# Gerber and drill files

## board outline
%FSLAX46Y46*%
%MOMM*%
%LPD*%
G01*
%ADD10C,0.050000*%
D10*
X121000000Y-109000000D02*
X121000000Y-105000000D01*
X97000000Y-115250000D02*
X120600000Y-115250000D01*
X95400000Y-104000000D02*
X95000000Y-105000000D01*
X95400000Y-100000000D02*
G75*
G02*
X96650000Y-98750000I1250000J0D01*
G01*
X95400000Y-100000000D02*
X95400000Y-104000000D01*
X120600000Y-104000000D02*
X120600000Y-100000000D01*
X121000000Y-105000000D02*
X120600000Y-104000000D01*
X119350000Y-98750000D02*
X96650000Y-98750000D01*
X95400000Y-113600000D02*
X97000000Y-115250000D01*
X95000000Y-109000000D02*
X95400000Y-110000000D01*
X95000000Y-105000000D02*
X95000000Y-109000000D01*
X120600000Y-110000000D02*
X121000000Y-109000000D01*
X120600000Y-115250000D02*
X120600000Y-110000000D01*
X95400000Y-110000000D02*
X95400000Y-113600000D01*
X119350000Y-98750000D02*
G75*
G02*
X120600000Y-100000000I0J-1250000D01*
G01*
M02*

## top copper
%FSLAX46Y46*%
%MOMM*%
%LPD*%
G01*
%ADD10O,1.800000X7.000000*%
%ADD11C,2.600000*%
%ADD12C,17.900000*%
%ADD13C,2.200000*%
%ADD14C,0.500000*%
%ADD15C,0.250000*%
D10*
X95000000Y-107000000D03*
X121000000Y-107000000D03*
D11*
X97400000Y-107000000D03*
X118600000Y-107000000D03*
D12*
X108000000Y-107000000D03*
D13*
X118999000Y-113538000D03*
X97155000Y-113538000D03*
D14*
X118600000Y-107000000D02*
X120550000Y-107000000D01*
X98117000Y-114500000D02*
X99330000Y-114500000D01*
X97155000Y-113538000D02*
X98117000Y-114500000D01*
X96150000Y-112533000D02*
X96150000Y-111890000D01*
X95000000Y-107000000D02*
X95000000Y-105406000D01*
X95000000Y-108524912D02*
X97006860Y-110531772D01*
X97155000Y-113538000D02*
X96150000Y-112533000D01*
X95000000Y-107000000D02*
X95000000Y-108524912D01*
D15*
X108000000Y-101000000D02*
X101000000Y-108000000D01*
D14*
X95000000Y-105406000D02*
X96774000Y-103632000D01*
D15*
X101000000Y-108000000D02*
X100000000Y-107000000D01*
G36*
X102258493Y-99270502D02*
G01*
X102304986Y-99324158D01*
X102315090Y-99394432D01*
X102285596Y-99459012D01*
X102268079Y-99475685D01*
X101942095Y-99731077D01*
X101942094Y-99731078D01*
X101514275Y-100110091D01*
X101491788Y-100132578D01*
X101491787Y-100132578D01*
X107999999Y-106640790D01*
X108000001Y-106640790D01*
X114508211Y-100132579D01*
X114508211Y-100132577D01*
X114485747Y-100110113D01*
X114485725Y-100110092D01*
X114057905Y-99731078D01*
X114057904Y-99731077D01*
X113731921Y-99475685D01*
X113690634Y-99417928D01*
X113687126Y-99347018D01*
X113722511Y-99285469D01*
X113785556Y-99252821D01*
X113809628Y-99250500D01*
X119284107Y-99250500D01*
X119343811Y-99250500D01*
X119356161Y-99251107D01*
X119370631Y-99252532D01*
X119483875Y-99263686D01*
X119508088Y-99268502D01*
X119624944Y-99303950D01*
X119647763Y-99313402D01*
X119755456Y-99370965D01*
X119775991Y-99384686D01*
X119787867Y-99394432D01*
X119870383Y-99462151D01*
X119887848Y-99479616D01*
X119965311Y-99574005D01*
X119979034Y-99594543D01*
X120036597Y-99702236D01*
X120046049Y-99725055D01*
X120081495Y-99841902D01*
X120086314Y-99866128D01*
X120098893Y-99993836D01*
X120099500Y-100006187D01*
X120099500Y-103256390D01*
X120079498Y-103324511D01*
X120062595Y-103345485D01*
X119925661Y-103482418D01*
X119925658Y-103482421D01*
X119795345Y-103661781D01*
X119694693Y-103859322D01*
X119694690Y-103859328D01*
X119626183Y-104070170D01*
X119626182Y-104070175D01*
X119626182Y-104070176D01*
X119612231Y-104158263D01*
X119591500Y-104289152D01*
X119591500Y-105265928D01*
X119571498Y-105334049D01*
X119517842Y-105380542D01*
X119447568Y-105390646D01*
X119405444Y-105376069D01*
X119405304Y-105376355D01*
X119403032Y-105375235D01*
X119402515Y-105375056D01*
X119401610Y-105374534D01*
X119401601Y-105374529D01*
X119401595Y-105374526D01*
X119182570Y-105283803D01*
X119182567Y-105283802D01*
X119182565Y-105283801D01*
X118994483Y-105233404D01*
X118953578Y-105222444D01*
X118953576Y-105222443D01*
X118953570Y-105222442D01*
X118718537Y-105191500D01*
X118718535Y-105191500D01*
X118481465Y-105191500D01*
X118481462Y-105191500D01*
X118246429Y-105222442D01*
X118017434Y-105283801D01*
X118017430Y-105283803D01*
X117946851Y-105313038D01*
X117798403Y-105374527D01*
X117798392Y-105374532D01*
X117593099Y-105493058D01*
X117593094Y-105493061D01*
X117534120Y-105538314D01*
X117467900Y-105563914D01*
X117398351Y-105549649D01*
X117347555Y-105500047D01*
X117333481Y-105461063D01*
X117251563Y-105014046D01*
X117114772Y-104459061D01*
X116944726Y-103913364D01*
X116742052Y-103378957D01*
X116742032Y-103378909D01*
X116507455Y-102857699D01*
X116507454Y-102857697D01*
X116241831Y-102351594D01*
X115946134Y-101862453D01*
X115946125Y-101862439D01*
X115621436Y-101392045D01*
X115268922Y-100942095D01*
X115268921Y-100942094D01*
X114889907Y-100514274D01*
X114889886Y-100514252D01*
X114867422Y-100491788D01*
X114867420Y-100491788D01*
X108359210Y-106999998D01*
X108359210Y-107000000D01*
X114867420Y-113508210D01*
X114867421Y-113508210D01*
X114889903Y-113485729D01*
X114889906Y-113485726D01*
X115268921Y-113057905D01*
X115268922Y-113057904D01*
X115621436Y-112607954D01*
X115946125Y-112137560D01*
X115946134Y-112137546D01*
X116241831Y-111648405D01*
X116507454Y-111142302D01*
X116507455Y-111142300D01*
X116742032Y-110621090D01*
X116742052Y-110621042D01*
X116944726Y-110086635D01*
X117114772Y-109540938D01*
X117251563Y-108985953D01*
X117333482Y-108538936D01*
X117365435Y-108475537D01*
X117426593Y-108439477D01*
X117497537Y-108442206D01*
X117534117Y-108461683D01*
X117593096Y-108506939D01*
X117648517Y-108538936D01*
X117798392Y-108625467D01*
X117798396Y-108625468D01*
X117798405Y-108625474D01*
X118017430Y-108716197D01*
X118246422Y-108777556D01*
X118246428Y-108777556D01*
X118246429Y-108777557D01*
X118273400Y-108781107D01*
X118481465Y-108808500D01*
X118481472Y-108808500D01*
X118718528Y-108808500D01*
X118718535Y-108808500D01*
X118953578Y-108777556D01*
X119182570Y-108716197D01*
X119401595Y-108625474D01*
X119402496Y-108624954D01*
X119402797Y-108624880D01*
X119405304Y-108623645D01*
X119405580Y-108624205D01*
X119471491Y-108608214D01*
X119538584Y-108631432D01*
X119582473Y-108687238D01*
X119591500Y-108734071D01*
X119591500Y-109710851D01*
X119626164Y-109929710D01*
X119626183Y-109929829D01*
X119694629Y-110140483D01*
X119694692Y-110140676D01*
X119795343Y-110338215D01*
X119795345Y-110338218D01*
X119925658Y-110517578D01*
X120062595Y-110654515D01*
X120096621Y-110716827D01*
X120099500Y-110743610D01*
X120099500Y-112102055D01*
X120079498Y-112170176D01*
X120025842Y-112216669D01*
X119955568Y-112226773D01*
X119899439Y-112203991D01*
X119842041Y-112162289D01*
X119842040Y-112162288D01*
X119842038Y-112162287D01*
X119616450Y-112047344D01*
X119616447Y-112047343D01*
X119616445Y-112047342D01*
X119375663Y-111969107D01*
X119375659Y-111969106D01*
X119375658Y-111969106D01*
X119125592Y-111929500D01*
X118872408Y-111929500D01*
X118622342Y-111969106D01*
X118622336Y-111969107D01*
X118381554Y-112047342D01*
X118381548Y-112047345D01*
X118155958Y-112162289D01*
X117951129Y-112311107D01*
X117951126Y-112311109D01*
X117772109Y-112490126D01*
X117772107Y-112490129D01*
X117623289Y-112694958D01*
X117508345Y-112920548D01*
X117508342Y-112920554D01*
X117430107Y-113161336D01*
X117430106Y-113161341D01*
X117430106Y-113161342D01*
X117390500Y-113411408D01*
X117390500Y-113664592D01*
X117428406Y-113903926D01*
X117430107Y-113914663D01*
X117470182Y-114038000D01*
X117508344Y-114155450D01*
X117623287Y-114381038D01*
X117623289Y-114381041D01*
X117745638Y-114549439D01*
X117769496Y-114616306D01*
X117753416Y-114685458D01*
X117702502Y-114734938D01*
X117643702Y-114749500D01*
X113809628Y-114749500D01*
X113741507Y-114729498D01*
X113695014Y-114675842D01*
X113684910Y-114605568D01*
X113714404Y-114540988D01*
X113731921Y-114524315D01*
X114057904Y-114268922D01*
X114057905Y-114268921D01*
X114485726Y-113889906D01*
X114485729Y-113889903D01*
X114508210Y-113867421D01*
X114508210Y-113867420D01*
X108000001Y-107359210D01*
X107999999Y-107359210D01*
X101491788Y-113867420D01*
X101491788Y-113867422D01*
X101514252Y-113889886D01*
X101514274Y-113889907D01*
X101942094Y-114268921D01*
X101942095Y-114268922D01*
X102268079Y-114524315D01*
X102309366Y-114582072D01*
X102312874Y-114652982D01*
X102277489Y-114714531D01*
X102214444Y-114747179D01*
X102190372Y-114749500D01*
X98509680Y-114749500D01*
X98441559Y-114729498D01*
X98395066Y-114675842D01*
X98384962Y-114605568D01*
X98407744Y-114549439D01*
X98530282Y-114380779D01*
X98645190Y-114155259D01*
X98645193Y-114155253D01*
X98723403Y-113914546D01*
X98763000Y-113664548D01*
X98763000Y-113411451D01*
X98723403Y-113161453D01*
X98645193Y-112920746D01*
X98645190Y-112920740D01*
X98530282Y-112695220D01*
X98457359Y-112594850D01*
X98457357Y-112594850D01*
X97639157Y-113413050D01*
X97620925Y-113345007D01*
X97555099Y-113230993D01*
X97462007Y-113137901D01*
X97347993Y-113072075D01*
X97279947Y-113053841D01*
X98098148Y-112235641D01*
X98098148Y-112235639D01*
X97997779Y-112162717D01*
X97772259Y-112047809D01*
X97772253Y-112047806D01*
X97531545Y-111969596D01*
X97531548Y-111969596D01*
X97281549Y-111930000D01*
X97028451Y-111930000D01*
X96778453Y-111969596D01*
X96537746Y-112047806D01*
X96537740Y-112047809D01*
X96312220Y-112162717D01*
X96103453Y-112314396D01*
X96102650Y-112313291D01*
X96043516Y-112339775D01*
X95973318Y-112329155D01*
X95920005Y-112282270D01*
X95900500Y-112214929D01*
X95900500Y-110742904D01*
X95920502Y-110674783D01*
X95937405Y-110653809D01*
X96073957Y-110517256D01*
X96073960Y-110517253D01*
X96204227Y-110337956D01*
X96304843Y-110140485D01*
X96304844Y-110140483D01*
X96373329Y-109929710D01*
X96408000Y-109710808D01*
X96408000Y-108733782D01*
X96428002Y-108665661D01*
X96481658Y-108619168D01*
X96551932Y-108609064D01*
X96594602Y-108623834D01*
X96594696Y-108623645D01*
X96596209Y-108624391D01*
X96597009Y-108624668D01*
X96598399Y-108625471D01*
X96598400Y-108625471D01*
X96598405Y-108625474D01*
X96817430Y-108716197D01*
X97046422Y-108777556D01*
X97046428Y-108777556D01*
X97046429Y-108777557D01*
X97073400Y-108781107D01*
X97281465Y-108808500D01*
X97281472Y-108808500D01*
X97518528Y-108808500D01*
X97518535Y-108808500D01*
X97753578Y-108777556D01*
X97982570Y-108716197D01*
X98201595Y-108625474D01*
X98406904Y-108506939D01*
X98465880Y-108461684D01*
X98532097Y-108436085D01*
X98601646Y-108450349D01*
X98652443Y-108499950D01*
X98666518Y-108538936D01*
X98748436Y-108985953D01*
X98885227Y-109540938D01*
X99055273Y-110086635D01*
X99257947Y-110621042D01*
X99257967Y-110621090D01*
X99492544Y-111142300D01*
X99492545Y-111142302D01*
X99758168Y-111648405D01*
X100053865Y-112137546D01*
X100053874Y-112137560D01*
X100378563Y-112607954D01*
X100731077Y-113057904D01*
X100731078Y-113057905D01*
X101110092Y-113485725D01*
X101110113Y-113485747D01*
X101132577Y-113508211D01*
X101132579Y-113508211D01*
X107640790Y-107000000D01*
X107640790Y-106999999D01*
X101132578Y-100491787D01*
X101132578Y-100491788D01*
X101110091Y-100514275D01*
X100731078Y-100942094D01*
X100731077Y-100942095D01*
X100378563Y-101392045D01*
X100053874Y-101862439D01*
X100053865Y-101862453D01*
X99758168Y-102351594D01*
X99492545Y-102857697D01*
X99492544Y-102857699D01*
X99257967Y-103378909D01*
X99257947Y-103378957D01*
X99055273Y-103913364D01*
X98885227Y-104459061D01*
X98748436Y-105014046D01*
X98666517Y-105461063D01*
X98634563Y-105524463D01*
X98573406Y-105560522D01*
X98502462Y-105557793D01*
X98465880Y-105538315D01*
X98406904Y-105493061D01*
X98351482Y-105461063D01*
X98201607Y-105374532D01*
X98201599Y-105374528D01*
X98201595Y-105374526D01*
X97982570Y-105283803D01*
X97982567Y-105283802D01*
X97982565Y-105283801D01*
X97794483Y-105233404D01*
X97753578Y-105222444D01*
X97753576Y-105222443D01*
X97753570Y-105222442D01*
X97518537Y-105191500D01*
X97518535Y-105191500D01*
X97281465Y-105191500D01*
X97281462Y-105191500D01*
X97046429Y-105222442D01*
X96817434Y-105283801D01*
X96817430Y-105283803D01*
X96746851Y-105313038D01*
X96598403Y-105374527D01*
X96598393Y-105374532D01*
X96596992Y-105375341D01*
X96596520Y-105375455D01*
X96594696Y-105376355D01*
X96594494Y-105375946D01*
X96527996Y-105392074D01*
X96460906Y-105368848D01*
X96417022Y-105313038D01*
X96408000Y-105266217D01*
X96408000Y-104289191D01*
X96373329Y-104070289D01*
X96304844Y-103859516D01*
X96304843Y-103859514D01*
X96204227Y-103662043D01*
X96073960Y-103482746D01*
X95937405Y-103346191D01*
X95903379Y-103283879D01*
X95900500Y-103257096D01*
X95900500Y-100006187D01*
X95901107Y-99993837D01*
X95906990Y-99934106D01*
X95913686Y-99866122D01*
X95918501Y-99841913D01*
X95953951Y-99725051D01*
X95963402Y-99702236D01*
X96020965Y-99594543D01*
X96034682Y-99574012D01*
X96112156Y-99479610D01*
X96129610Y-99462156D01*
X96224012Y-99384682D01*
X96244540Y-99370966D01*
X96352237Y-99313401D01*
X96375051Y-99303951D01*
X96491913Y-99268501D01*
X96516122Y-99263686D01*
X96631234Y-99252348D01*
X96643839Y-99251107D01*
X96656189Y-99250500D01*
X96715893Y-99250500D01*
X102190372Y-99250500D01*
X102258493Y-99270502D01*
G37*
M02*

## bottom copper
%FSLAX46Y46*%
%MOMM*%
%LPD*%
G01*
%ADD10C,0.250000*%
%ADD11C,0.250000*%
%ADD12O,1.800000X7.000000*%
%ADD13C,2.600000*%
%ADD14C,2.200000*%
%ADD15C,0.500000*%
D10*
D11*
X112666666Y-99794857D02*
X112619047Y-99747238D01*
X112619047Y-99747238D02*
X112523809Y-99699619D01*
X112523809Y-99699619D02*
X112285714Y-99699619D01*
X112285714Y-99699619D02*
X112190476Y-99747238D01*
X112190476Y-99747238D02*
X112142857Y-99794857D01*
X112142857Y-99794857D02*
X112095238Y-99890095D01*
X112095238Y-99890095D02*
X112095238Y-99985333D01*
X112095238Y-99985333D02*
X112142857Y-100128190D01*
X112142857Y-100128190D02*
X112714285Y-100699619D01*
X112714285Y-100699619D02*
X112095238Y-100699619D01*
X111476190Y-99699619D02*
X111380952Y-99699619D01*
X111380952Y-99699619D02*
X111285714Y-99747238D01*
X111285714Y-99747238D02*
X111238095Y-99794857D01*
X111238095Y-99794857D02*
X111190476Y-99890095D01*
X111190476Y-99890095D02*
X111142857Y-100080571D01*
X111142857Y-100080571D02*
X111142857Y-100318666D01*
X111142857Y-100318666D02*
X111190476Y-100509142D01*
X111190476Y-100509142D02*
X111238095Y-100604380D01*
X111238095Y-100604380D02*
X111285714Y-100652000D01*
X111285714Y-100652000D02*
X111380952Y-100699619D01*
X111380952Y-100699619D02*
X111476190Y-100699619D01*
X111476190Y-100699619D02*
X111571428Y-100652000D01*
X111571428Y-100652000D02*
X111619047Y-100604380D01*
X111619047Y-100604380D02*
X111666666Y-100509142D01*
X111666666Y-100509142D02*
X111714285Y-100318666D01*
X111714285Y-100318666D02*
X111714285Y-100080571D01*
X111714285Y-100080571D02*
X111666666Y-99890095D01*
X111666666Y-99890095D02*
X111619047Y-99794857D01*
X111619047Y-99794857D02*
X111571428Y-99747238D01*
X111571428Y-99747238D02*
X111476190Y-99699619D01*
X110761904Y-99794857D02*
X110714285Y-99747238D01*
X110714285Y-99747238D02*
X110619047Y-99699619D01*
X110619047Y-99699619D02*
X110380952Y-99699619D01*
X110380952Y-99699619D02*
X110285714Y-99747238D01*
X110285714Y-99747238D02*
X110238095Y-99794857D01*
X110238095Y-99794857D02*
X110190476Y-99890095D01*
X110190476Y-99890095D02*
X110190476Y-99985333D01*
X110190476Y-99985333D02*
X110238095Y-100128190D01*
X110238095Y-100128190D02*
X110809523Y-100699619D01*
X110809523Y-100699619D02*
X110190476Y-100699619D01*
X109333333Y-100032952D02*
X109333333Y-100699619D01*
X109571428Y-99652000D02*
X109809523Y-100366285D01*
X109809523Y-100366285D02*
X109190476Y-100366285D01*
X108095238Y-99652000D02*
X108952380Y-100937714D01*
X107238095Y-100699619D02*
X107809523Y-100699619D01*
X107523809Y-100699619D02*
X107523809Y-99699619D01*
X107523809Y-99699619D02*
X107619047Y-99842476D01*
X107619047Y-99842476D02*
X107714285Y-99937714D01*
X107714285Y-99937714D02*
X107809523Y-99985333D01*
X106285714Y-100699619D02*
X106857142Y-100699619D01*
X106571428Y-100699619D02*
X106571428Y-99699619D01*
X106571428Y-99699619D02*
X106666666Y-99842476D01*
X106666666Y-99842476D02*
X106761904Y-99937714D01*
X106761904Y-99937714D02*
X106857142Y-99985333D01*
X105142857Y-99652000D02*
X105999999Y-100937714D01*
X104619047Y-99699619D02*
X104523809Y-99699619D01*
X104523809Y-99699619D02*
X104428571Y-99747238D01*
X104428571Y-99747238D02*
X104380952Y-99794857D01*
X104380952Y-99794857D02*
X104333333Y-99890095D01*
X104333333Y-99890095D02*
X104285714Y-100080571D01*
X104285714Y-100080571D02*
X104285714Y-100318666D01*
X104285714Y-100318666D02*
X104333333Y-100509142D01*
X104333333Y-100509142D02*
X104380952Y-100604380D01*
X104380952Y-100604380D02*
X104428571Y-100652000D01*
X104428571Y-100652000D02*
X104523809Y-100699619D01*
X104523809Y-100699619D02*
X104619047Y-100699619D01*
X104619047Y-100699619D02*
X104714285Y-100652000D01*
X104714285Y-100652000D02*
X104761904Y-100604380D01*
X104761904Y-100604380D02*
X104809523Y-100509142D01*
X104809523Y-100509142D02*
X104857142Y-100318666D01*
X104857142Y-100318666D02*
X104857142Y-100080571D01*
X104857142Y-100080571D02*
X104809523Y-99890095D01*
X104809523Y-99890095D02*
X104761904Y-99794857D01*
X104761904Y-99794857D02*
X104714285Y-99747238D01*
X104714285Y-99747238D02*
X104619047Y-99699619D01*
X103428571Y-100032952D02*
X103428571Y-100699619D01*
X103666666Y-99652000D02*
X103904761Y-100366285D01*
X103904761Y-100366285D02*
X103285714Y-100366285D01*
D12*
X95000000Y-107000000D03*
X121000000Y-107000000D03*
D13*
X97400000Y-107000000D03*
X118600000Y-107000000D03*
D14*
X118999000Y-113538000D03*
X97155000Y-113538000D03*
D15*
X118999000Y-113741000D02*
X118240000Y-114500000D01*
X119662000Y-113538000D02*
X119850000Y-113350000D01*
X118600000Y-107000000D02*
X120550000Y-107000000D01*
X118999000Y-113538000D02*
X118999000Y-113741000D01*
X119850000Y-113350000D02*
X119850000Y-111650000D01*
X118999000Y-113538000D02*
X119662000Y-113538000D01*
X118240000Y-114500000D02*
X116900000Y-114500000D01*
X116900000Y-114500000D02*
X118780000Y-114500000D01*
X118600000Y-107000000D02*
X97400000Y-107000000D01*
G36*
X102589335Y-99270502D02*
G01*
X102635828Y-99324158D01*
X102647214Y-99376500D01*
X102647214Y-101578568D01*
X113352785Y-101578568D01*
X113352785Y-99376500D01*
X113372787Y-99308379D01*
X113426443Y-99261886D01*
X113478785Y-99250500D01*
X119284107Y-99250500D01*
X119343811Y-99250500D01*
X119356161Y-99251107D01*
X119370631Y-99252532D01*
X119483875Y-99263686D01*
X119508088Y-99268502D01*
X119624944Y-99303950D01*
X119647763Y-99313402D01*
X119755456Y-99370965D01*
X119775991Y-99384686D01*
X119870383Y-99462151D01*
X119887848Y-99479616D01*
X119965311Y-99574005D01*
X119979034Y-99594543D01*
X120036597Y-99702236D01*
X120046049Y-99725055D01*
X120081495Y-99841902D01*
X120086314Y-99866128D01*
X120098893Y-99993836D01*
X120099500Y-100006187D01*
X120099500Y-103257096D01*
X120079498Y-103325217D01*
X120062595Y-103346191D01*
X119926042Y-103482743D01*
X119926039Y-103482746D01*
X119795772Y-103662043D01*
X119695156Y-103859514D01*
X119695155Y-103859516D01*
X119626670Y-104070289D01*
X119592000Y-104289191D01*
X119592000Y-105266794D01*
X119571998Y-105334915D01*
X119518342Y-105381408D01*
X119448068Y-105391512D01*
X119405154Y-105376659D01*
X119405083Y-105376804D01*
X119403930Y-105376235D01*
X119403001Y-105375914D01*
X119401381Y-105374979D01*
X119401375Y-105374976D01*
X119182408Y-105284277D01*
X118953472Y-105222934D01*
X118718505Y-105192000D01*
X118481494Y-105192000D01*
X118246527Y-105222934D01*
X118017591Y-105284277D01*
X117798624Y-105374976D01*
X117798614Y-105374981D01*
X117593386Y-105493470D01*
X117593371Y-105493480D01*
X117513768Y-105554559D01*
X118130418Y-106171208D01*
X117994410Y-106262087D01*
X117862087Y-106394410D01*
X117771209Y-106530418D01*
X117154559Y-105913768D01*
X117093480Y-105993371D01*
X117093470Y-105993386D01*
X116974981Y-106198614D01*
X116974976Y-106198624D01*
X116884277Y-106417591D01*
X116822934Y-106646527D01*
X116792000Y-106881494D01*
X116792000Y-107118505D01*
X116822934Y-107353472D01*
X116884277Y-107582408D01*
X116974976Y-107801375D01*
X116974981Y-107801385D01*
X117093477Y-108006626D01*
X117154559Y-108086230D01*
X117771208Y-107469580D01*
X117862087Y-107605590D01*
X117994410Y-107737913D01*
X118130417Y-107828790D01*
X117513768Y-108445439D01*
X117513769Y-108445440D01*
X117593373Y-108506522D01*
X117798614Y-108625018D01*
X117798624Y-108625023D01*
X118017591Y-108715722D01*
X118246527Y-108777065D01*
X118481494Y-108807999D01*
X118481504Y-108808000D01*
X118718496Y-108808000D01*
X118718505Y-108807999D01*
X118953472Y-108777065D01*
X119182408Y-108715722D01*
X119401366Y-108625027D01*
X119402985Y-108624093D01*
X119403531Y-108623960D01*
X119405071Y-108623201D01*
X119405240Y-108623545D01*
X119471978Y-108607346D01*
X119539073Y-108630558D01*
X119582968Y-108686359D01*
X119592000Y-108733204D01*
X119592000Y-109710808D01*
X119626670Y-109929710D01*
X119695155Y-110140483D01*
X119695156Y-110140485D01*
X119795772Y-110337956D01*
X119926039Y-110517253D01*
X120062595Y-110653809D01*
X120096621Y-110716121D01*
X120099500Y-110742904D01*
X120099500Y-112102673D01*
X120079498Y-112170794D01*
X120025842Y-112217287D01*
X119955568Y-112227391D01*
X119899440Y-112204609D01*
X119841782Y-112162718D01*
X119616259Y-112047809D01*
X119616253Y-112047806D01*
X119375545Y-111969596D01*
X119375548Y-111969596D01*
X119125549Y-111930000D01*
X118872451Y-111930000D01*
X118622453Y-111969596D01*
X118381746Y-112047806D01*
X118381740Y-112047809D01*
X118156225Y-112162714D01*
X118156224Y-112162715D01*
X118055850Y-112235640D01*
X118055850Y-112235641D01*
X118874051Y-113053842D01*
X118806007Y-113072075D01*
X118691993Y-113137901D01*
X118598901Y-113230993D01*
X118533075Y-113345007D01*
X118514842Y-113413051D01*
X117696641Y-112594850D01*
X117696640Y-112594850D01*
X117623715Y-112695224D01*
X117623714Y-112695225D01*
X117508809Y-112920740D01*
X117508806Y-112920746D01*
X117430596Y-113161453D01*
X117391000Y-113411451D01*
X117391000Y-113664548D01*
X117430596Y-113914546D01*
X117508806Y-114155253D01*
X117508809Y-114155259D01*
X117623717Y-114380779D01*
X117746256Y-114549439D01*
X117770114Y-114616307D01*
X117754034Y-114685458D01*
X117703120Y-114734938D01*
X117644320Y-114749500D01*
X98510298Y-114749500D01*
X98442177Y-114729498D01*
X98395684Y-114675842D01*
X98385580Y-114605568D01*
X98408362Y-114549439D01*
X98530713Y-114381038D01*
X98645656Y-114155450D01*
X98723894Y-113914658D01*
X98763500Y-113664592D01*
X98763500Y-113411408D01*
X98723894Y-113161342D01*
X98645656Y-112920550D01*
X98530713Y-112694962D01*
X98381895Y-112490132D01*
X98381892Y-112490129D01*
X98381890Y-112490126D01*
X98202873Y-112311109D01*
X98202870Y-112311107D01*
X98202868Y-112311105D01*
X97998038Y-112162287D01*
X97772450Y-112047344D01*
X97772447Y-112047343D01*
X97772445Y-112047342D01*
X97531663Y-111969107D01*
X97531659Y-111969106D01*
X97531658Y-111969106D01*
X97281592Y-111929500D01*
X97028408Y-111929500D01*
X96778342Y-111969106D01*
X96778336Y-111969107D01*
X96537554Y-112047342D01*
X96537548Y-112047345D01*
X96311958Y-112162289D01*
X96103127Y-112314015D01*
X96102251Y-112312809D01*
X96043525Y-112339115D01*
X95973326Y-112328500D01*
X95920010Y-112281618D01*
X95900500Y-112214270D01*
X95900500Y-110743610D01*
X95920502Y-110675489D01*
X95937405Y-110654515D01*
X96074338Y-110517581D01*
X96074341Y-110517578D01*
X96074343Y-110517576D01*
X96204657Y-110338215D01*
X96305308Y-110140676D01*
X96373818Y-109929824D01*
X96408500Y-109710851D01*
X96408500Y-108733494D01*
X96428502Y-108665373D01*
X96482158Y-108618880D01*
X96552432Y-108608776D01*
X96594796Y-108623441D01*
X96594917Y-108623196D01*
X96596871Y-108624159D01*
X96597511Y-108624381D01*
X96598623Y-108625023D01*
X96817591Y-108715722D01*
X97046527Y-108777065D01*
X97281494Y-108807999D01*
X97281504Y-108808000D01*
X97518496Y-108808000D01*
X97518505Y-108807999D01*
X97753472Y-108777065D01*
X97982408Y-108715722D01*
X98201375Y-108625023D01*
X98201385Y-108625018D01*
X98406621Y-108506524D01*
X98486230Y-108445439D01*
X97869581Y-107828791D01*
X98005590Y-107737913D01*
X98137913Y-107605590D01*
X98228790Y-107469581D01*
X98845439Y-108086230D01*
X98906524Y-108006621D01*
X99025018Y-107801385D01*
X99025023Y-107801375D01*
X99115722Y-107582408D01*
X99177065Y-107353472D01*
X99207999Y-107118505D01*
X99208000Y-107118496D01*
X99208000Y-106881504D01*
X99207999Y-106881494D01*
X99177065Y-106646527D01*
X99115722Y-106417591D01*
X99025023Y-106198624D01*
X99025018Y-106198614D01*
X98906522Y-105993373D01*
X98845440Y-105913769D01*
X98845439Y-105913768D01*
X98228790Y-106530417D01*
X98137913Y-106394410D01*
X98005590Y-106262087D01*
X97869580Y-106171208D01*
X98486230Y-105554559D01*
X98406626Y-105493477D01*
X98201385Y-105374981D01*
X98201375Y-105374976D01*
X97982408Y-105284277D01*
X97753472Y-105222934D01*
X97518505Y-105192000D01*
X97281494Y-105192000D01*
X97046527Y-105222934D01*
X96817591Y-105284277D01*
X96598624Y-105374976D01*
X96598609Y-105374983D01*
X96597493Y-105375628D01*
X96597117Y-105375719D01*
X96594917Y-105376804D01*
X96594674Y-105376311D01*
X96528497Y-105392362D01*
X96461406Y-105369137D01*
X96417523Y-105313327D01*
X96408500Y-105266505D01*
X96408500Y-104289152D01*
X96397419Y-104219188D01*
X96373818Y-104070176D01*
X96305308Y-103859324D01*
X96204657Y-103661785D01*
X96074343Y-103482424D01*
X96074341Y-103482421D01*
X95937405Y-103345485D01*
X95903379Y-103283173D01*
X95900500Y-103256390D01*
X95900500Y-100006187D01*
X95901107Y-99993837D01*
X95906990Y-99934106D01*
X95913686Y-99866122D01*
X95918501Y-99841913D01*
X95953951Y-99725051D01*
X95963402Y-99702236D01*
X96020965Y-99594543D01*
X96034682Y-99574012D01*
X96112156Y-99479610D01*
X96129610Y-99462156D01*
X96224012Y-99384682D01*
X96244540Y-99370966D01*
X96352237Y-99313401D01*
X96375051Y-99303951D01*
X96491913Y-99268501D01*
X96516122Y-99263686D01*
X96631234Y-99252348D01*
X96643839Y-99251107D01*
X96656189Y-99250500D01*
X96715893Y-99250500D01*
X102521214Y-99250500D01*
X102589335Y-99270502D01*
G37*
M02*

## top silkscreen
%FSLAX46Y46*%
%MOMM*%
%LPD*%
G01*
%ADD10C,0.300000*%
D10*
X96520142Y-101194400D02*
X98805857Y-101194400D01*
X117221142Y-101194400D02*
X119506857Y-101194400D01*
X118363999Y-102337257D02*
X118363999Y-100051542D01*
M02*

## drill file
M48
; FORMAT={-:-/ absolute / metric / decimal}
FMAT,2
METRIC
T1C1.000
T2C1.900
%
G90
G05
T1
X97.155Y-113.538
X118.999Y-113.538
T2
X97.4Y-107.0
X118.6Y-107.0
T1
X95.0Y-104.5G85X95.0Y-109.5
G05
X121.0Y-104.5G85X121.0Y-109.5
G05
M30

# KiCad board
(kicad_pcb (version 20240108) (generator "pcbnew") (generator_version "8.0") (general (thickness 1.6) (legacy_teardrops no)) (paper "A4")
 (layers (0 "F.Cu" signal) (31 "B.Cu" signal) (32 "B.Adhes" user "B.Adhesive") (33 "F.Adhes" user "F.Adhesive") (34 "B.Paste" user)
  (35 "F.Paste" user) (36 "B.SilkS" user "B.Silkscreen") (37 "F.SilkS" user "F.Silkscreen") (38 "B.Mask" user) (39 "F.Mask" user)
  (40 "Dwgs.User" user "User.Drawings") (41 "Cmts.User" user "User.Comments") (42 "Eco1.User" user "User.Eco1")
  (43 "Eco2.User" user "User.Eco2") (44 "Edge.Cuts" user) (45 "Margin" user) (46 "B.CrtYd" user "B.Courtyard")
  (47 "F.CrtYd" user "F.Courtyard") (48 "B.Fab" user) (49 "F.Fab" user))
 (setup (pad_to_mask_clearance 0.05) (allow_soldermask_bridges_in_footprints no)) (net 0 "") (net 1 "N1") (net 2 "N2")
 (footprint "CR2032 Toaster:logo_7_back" (layer "F.Cu") (at 114 106.25)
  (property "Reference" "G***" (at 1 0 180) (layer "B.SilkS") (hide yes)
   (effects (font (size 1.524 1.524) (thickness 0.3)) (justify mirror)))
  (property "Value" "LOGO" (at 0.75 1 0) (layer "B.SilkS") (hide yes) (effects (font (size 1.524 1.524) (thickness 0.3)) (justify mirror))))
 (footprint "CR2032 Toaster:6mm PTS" (layer "F.Cu") (at 95 107)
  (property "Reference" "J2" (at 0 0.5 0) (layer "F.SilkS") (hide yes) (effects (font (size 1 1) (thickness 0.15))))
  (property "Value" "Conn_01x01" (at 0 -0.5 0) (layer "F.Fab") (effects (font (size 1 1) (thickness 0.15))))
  (pad "1" thru_hole oval (at 0 0) (size 1.8 7) (drill oval 1 6) (layers "*.Cu" "*.Mask") (remove_unused_layers no) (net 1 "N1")))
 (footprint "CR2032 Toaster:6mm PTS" (layer "F.Cu") (at 121 107)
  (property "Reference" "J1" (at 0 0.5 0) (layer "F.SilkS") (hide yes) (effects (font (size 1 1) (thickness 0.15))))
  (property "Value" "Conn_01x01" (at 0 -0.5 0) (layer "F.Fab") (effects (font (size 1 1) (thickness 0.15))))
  (pad "1" thru_hole oval (at 0 0) (size 1.8 7) (drill oval 1 6) (layers "*.Cu" "*.Mask") (remove_unused_layers no) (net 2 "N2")))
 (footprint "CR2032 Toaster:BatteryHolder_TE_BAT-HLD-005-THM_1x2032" (layer "F.Cu") (at 108 107)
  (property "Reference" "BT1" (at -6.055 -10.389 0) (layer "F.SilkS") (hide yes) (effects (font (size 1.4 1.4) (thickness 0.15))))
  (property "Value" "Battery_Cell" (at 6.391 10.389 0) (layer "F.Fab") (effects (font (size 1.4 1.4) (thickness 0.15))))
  (pad "1" thru_hole circle (at -10.6 0) (size 2.6 2.6) (drill 1.9) (layers "*.Cu" "*.Mask") (remove_unused_layers no) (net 2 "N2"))
  (pad "1" thru_hole circle (at 10.6 0) (size 2.6 2.6) (drill 1.9) (layers "*.Cu" "*.Mask") (remove_unused_layers no) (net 2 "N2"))
  (pad "2" smd circle (at 0 0) (size 17.9 17.9) (layers "F.Cu" "F.Paste" "F.Mask") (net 1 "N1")))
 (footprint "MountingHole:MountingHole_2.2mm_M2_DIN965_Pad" (layer "F.Cu") (at 118.999 113.538)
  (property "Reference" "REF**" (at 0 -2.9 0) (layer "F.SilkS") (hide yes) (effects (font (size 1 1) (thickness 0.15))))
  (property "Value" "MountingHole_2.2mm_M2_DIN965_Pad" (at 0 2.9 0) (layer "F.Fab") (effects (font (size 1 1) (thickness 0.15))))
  (pad "1" thru_hole circle (at 0 0) (size 2.2 2.2) (drill 1) (layers "*.Cu" "*.Mask") (remove_unused_layers no) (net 2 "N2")))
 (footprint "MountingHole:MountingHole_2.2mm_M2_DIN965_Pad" (layer "F.Cu") (at 97.155 113.538)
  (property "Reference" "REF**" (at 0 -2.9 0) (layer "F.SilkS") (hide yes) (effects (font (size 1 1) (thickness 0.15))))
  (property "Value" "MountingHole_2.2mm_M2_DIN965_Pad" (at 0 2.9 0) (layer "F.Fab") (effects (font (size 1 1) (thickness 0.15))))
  (pad "1" thru_hole circle (at 0 0) (size 2.2 2.2) (drill 1) (layers "*.Cu" "*.Mask") (remove_unused_layers no) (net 1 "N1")))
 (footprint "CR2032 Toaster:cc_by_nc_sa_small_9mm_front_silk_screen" (layer "B.Cu") (at 107.95 113.5 180)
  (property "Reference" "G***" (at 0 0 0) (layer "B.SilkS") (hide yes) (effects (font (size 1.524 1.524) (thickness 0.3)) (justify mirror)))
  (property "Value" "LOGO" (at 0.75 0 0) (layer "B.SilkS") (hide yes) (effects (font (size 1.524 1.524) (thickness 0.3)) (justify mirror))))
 (gr_line (start 121 109) (end 121 105) (stroke (width 0.05) (type solid)) (layer "Edge.Cuts"))
 (gr_line (start 97 115.25) (end 120.6 115.25) (stroke (width 0.05) (type solid)) (layer "Edge.Cuts"))
 (gr_line (start 95.4 104) (end 95 105) (stroke (width 0.05) (type solid)) (layer "Edge.Cuts"))
 (gr_arc (start 95.4 100) (mid 95.766117 99.116117) (end 96.65 98.75) (stroke (width 0.05) (type solid)) (layer "Edge.Cuts"))
 (gr_line (start 95.4 100) (end 95.4 104) (stroke (width 0.05) (type solid)) (layer "Edge.Cuts"))
 (gr_line (start 120.6 104) (end 120.6 100) (stroke (width 0.05) (type solid)) (layer "Edge.Cuts"))
 (gr_line (start 121 105) (end 120.6 104) (stroke (width 0.05) (type solid)) (layer "Edge.Cuts"))
 (gr_line (start 119.35 98.75) (end 96.65 98.75) (stroke (width 0.05) (type solid)) (layer "Edge.Cuts"))
 (gr_line (start 95.4 113.6) (end 97 115.25) (stroke (width 0.05) (type solid)) (layer "Edge.Cuts"))
 (gr_line (start 95 109) (end 95.4 110) (stroke (width 0.05) (type solid)) (layer "Edge.Cuts"))
 (gr_line (start 95 105) (end 95 109) (stroke (width 0.05) (type solid)) (layer "Edge.Cuts"))
 (gr_line (start 120.6 110) (end 121 109) (stroke (width 0.05) (type solid)) (layer "Edge.Cuts"))
 (gr_line (start 120.6 115.25) (end 120.6 110) (stroke (width 0.05) (type solid)) (layer "Edge.Cuts"))
 (gr_line (start 95.4 110) (end 95.4 113.6) (stroke (width 0.05) (type solid)) (layer "Edge.Cuts"))
 (gr_arc (start 119.35 98.75) (mid 120.233883 99.116117) (end 120.6 100) (stroke (width 0.05) (type solid)) (layer "Edge.Cuts"))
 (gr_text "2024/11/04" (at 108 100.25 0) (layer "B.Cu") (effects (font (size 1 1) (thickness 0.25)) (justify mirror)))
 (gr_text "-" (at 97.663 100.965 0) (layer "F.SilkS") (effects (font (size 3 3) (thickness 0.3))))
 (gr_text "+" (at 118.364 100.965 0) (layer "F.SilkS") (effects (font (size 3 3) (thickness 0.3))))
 (segment (start 118.6 107) (end 120.55 107) (width 0.5) (layer "F.Cu") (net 2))
 (segment (start 118.999 113.741) (end 118.24 114.5) (width 0.5) (layer "B.Cu") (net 2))
 (segment (start 119.662 113.538) (end 119.85 113.35) (width 0.5) (layer "B.Cu") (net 2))
 (segment (start 118.6 107) (end 120.55 107) (width 0.5) (layer "B.Cu") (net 2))
 (segment (start 118.999 113.538) (end 118.999 113.741) (width 0.5) (layer "B.Cu") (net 2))
 (segment (start 119.85 113.35) (end 119.85 111.65) (width 0.5) (layer "B.Cu") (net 2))
 (segment (start 118.999 113.538) (end 119.662 113.538) (width 0.5) (layer "B.Cu") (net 2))
 (segment (start 118.24 114.5) (end 116.9 114.5) (width 0.5) (layer "B.Cu") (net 2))
 (segment (start 116.9 114.5) (end 118.78 114.5) (width 0.5) (layer "B.Cu") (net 2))
 (segment (start 118.6 107) (end 97.4 107) (width 0.5) (layer "B.Cu") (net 2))
 (segment (start 98.117 114.5) (end 99.33 114.5) (width 0.5) (layer "F.Cu") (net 1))
 (segment (start 97.155 113.538) (end 98.117 114.5) (width 0.5) (layer "F.Cu") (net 1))
 (segment (start 96.15 112.533) (end 96.15 111.89) (width 0.5) (layer "F.Cu") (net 1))
 (segment (start 95 107) (end 95 105.406) (width 0.5) (layer "F.Cu") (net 1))
 (segment (start 95 108.524912) (end 97.00686 110.531772) (width 0.5) (layer "F.Cu") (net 1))
 (segment (start 97.155 113.538) (end 96.15 112.533) (width 0.5) (layer "F.Cu") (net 1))
 (segment (start 95 107) (end 95 108.524912) (width 0.5) (layer "F.Cu") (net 1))
 (segment (start 108 101) (end 101 108) (width 0.25) (layer "F.Cu") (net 1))
 (segment (start 95 105.406) (end 96.774 103.632) (width 0.5) (layer "F.Cu") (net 1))
 (segment (start 101 108) (end 100 107) (width 0.25) (layer "F.Cu") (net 1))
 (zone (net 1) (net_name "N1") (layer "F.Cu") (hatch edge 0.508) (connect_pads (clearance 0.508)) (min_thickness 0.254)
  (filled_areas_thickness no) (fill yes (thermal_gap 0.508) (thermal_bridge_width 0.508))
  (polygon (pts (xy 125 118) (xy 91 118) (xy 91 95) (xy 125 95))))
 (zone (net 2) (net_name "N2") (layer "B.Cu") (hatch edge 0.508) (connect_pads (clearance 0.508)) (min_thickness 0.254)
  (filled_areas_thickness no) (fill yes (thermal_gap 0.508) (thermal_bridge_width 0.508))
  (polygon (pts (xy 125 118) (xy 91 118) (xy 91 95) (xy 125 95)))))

